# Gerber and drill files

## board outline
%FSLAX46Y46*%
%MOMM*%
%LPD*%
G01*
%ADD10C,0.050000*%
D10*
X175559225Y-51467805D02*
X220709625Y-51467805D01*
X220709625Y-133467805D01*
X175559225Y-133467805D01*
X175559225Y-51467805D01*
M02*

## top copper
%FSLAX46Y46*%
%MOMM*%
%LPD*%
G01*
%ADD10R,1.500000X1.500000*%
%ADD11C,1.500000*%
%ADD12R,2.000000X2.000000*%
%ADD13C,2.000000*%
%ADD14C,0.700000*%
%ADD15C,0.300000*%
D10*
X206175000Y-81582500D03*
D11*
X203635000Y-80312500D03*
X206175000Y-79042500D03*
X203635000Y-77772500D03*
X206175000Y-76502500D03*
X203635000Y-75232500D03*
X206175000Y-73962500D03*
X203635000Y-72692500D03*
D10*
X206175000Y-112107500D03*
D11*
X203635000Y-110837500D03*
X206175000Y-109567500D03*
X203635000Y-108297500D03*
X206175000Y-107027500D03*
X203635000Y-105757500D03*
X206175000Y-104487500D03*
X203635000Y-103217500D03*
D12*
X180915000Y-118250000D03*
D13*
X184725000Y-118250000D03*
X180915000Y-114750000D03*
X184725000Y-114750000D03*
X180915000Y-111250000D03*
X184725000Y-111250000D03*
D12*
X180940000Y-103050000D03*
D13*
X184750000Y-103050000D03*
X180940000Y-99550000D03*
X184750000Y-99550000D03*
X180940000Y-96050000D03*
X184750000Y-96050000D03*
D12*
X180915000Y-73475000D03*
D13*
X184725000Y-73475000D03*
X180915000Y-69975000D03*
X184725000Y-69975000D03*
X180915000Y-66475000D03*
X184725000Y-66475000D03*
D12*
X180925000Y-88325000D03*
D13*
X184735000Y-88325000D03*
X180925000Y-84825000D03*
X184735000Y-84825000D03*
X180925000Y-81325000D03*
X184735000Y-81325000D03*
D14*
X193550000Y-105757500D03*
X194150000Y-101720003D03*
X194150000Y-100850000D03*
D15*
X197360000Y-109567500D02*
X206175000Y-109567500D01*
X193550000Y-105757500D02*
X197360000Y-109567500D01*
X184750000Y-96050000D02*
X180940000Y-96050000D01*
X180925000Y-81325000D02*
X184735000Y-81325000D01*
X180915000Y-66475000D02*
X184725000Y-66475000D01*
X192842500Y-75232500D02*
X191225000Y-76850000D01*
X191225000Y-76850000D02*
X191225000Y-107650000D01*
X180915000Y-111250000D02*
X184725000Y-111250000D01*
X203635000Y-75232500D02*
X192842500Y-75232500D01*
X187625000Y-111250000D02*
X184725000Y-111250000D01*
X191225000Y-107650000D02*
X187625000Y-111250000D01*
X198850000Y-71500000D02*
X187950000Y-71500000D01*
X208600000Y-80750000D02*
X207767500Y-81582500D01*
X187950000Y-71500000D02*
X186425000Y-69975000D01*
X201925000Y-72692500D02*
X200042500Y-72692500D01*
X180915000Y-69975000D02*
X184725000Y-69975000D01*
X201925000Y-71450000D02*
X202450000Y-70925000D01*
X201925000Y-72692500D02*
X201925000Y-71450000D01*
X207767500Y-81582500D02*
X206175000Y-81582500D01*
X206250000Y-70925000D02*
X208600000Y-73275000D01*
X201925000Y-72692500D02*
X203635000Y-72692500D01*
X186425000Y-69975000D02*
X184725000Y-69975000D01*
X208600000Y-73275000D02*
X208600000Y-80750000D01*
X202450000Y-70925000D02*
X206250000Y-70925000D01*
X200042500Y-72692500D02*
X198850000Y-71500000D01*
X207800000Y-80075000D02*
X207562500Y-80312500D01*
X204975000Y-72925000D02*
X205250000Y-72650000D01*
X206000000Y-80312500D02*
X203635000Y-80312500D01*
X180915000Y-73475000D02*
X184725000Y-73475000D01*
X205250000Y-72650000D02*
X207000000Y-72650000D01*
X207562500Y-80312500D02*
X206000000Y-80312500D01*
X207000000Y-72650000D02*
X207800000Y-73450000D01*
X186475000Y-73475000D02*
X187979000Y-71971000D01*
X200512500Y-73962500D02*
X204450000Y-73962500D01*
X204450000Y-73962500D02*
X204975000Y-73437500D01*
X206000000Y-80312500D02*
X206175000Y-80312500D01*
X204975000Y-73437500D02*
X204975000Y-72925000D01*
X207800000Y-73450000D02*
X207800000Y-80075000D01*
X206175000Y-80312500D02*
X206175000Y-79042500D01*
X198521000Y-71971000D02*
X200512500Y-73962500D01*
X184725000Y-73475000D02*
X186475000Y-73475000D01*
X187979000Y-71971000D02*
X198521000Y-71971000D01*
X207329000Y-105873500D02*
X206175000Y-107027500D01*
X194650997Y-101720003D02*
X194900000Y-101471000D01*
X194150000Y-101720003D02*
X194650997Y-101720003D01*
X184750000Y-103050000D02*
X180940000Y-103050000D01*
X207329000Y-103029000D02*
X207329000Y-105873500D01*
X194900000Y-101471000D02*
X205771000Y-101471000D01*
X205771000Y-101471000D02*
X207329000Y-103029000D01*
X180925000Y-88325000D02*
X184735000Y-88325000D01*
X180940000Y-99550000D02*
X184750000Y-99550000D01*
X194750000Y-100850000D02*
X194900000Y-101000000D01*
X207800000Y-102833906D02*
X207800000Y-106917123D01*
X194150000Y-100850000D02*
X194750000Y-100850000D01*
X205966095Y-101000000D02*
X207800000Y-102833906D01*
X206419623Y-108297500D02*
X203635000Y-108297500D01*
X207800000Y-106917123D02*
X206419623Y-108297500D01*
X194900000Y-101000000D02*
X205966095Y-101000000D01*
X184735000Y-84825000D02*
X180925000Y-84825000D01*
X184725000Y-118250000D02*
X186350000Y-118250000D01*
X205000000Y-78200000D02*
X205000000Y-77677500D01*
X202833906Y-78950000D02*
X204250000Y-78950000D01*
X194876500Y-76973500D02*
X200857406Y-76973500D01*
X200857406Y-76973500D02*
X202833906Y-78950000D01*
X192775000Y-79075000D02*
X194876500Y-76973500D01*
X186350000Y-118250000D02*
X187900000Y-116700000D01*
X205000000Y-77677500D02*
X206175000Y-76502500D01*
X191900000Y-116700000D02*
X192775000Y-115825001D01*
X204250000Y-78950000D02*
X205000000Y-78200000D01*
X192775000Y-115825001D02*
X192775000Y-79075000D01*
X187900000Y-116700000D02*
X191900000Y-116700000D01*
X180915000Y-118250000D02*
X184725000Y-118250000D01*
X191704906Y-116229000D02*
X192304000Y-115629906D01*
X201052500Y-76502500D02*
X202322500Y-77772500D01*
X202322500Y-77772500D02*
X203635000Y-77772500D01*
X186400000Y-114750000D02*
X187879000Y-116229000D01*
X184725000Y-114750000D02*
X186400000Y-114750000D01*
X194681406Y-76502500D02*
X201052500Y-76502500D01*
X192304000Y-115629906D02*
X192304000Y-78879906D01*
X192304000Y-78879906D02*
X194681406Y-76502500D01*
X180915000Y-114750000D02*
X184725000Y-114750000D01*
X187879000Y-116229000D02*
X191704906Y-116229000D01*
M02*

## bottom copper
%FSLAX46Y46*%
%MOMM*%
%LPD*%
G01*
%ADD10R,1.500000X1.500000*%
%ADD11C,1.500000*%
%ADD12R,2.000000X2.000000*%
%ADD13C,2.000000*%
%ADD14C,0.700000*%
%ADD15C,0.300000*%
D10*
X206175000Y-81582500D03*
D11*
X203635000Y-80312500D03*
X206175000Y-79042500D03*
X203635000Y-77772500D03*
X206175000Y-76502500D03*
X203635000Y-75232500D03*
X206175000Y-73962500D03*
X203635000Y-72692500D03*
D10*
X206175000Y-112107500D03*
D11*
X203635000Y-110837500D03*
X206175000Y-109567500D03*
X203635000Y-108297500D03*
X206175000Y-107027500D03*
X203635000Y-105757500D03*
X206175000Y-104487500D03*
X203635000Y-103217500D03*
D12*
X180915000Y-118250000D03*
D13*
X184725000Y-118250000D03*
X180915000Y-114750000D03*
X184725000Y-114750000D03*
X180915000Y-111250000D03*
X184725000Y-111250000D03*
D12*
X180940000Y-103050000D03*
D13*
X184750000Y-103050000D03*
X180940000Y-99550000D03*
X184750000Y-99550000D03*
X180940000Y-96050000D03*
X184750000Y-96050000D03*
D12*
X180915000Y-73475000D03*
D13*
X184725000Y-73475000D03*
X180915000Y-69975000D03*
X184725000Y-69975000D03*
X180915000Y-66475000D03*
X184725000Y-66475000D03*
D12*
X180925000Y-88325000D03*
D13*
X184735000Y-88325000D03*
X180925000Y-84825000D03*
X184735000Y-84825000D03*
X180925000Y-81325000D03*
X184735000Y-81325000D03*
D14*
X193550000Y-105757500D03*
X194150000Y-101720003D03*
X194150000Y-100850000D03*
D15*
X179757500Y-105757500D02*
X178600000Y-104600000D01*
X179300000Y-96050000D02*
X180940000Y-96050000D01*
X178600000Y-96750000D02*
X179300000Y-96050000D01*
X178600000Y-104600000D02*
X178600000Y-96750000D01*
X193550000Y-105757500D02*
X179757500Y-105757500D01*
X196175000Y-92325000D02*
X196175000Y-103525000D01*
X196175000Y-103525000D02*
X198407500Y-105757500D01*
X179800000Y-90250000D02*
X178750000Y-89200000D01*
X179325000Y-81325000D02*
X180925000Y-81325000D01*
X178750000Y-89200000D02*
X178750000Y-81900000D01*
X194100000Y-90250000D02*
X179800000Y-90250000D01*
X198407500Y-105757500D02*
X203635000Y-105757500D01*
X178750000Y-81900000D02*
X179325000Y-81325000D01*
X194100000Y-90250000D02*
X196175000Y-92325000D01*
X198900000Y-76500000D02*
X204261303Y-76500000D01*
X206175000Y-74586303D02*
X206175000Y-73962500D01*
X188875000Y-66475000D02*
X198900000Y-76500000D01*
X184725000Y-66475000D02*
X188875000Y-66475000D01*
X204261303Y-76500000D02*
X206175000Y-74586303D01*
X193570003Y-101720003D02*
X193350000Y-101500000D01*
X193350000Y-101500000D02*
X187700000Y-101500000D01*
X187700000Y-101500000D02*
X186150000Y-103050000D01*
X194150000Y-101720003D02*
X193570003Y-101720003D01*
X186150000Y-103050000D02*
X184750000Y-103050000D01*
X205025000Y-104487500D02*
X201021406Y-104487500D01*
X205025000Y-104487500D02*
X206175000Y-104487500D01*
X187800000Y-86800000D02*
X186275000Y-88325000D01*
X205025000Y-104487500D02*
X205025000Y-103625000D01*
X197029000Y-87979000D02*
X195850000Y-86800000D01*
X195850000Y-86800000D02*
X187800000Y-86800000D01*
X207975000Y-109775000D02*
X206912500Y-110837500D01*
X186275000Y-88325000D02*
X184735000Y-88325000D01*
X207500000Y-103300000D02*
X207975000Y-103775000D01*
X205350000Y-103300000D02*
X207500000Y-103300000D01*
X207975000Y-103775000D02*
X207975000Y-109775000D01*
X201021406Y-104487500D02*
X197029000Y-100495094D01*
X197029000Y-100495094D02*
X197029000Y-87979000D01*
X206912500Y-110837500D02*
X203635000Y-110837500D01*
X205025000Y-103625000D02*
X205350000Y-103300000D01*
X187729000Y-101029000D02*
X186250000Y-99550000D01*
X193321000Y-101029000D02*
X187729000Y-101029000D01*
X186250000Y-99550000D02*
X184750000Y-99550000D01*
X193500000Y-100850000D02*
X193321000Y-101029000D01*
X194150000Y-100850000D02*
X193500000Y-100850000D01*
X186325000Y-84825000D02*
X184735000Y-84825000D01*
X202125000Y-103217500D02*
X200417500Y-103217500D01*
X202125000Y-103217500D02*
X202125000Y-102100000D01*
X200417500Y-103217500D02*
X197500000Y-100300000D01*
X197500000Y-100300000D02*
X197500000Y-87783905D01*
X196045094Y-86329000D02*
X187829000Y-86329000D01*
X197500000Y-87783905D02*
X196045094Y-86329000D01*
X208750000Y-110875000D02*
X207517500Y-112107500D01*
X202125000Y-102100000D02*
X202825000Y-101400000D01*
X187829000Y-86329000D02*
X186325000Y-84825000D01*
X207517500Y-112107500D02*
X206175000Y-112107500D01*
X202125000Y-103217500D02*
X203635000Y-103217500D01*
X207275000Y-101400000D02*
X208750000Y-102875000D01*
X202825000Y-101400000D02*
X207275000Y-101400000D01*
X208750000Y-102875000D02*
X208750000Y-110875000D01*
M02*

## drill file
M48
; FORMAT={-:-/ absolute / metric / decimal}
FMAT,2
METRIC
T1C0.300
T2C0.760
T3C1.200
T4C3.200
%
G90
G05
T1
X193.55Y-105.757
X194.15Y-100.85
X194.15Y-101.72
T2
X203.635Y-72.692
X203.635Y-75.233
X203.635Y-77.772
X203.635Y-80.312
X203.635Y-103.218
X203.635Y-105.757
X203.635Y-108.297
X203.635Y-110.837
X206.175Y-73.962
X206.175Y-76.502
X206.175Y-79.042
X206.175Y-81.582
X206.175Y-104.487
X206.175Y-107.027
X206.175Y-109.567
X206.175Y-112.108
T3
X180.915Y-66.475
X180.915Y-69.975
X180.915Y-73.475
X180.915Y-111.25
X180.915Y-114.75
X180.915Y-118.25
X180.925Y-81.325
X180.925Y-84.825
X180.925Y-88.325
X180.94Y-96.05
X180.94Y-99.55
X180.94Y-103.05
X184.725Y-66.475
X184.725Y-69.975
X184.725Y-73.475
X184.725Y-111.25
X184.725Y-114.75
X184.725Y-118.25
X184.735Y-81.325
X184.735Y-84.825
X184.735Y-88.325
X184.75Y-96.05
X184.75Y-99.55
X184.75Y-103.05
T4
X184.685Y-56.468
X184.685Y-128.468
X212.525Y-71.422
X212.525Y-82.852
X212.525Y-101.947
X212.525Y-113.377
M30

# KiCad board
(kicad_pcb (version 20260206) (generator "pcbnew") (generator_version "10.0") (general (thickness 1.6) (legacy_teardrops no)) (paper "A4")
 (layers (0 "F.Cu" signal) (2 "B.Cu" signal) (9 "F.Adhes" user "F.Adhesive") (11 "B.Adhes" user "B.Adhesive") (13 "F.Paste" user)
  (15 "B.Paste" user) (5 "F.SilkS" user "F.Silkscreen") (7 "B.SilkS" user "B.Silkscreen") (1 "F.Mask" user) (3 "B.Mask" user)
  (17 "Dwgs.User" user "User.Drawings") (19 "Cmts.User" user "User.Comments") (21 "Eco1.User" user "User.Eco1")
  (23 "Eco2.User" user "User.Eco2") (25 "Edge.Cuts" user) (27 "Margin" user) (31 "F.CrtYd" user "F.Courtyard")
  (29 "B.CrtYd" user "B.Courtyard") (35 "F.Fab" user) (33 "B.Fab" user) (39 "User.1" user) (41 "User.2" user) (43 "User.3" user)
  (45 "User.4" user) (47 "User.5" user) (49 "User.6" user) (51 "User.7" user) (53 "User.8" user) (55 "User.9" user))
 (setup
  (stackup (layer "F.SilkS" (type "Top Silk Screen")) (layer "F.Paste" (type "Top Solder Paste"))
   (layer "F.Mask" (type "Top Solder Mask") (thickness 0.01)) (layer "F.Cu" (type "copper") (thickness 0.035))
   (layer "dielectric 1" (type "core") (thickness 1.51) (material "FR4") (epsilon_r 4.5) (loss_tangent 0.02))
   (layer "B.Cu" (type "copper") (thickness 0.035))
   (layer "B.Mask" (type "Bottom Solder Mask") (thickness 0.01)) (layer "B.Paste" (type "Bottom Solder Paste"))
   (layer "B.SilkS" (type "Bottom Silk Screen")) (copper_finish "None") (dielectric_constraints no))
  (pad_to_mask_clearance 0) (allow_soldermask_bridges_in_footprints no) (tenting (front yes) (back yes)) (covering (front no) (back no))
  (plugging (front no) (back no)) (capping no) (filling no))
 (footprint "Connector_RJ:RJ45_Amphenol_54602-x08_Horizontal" (layer "F.Cu") (at 206.175 81.5825 90)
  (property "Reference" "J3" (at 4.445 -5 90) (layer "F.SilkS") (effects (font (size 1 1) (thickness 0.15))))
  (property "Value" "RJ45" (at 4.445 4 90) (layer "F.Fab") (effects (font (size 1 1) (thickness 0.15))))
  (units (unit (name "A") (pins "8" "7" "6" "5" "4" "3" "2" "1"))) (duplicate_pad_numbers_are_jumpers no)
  (pad "" np_thru_hole circle (at -1.27 6.35 90) (size 3.2 3.2) (drill 3.2) (layers "*.Cu" "*.Mask"))
  (pad "" np_thru_hole circle (at 10.16 6.35 90) (size 3.2 3.2) (drill 3.2) (layers "*.Cu" "*.Mask"))
  (pad "1" thru_hole rect (at 0 0 90) (size 1.5 1.5) (drill 0.76) (layers "*.Cu" "*.Mask") (remove_unused_layers no) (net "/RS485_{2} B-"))
  (pad "2" thru_hole circle (at 1.27 -2.54 90) (size 1.5 1.5) (drill 0.76) (layers "*.Cu" "*.Mask") (remove_unused_layers no)
   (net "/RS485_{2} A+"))
  (pad "3" thru_hole circle (at 2.54 0 90) (size 1.5 1.5) (drill 0.76) (layers "*.Cu" "*.Mask") (remove_unused_layers no)
   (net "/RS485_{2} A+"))
  (pad "4" thru_hole circle (at 3.81 -2.54 90) (size 1.5 1.5) (drill 0.76) (layers "*.Cu" "*.Mask") (remove_unused_layers no)
   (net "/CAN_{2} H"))
  (pad "5" thru_hole circle (at 5.08 0 90) (size 1.5 1.5) (drill 0.76) (layers "*.Cu" "*.Mask") (remove_unused_layers no) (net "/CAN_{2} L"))
  (pad "6" thru_hole circle (at 6.35 -2.54 90) (size 1.5 1.5) (drill 0.76) (layers "*.Cu" "*.Mask") (remove_unused_layers no)
   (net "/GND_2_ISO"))
  (pad "7" thru_hole circle (at 7.62 0 90) (size 1.5 1.5) (drill 0.76) (layers "*.Cu" "*.Mask") (remove_unused_layers no) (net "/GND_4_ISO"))
  (pad "8" thru_hole circle (at 8.89 -2.54 90) (size 1.5 1.5) (drill 0.76) (layers "*.Cu" "*.Mask") (remove_unused_layers no)
   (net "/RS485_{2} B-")))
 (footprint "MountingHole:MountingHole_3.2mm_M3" (layer "F.Cu") (at 184.684625 56.467805)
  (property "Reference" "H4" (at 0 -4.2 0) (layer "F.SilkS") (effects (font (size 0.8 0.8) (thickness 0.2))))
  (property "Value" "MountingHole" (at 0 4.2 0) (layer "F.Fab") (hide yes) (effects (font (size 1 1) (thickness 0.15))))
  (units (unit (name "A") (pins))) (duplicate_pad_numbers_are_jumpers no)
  (pad "" np_thru_hole circle (at 0 0) (size 3.2 3.2) (drill 3.2) (layers "*.Cu" "*.Mask")))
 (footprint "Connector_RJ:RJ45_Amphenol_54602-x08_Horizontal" (layer "F.Cu") (at 206.175 112.1075 90)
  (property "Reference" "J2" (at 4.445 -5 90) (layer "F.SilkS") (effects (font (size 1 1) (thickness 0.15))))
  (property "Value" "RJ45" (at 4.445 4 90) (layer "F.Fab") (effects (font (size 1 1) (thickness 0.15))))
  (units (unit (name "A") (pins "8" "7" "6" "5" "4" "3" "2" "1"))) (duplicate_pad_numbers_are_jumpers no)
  (pad "" np_thru_hole circle (at -1.27 6.35 90) (size 3.2 3.2) (drill 3.2) (layers "*.Cu" "*.Mask"))
  (pad "" np_thru_hole circle (at 10.16 6.35 90) (size 3.2 3.2) (drill 3.2) (layers "*.Cu" "*.Mask"))
  (pad "1" thru_hole rect (at 0 0 90) (size 1.5 1.5) (drill 0.76) (layers "*.Cu" "*.Mask") (remove_unused_layers no) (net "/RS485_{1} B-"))
  (pad "2" thru_hole circle (at 1.27 -2.54 90) (size 1.5 1.5) (drill 0.76) (layers "*.Cu" "*.Mask") (remove_unused_layers no)
   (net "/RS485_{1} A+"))
  (pad "3" thru_hole circle (at 2.54 0 90) (size 1.5 1.5) (drill 0.76) (layers "*.Cu" "*.Mask") (remove_unused_layers no) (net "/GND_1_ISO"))
  (pad "4" thru_hole circle (at 3.81 -2.54 90) (size 1.5 1.5) (drill 0.76) (layers "*.Cu" "*.Mask") (remove_unused_layers no)
   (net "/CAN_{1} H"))
  (pad "5" thru_hole circle (at 5.08 0 90) (size 1.5 1.5) (drill 0.76) (layers "*.Cu" "*.Mask") (remove_unused_layers no) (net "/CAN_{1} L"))
  (pad "6" thru_hole circle (at 6.35 -2.54 90) (size 1.5 1.5) (drill 0.76) (layers "*.Cu" "*.Mask") (remove_unused_layers no)
   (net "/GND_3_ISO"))
  (pad "7" thru_hole circle (at 7.62 0 90) (size 1.5 1.5) (drill 0.76) (layers "*.Cu" "*.Mask") (remove_unused_layers no)
   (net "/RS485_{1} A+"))
  (pad "8" thru_hole circle (at 8.89 -2.54 90) (size 1.5 1.5) (drill 0.76) (layers "*.Cu" "*.Mask") (remove_unused_layers no)
   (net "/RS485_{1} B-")))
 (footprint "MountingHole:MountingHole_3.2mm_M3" (layer "F.Cu") (at 184.684625 128.467805)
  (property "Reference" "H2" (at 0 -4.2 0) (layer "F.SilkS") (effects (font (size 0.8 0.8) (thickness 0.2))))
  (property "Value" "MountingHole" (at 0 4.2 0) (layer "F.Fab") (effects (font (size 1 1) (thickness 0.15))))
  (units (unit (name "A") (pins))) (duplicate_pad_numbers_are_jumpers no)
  (pad "" np_thru_hole circle (at 0 0) (size 3.2 3.2) (drill 3.2) (layers "*.Cu" "*.Mask")))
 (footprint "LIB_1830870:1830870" (layer "B.Cu") (at 180.915 118.25 90)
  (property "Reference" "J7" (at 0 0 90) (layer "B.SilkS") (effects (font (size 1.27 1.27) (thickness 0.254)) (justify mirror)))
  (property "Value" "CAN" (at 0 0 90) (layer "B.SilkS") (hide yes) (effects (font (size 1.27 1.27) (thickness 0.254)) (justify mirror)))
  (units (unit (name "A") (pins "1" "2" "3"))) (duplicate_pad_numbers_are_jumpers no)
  (pad "1" thru_hole rect (at 0 0 90) (size 2 2) (drill 1.2) (layers "*.Cu" "*.Mask") (remove_unused_layers no) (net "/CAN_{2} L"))
  (pad "1" thru_hole circle (at 0 3.81 90) (size 2 2) (drill 1.2) (layers "*.Cu" "*.Mask") (remove_unused_layers no) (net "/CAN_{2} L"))
  (pad "2" thru_hole circle (at 3.5 0 90) (size 2 2) (drill 1.2) (layers "*.Cu" "*.Mask") (remove_unused_layers no) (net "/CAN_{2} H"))
  (pad "2" thru_hole circle (at 3.5 3.81 90) (size 2 2) (drill 1.2) (layers "*.Cu" "*.Mask") (remove_unused_layers no) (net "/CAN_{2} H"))
  (pad "3" thru_hole circle (at 7 0 90) (size 2 2) (drill 1.2) (layers "*.Cu" "*.Mask") (remove_unused_layers no) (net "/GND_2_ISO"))
  (pad "3" thru_hole circle (at 7 3.81 90) (size 2 2) (drill 1.2) (layers "*.Cu" "*.Mask") (remove_unused_layers no) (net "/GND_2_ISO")))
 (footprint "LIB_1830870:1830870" (layer "B.Cu") (at 180.94 103.05 90)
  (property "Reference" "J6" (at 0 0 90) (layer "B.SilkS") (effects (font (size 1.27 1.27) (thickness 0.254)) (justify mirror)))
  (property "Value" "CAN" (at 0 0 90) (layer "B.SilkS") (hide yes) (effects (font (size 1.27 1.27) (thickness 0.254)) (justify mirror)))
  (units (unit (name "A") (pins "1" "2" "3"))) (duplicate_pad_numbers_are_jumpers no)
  (pad "1" thru_hole rect (at 0 0 90) (size 2 2) (drill 1.2) (layers "*.Cu" "*.Mask") (remove_unused_layers no) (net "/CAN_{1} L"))
  (pad "1" thru_hole circle (at 0 3.81 90) (size 2 2) (drill 1.2) (layers "*.Cu" "*.Mask") (remove_unused_layers no) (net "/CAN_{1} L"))
  (pad "2" thru_hole circle (at 3.5 0 90) (size 2 2) (drill 1.2) (layers "*.Cu" "*.Mask") (remove_unused_layers no) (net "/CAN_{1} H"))
  (pad "2" thru_hole circle (at 3.5 3.81 90) (size 2 2) (drill 1.2) (layers "*.Cu" "*.Mask") (remove_unused_layers no) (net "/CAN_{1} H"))
  (pad "3" thru_hole circle (at 7 0 90) (size 2 2) (drill 1.2) (layers "*.Cu" "*.Mask") (remove_unused_layers no) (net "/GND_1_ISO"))
  (pad "3" thru_hole circle (at 7 3.81 90) (size 2 2) (drill 1.2) (layers "*.Cu" "*.Mask") (remove_unused_layers no) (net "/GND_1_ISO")))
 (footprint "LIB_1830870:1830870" (layer "B.Cu") (at 180.915 73.475 90)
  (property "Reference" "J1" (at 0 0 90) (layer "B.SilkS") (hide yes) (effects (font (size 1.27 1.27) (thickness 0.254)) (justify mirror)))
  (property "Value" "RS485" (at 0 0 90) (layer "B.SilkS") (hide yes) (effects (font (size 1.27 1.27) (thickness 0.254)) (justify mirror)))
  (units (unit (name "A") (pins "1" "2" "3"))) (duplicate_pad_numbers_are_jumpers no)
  (pad "1" thru_hole rect (at 0 0 90) (size 2 2) (drill 1.2) (layers "*.Cu" "*.Mask") (remove_unused_layers no) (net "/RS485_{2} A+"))
  (pad "1" thru_hole circle (at 0 3.81 90) (size 2 2) (drill 1.2) (layers "*.Cu" "*.Mask") (remove_unused_layers no) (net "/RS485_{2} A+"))
  (pad "2" thru_hole circle (at 3.5 0 90) (size 2 2) (drill 1.2) (layers "*.Cu" "*.Mask") (remove_unused_layers no) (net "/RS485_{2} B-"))
  (pad "2" thru_hole circle (at 3.5 3.81 90) (size 2 2) (drill 1.2) (layers "*.Cu" "*.Mask") (remove_unused_layers no) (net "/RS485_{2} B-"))
  (pad "3" thru_hole circle (at 7 0 90) (size 2 2) (drill 1.2) (layers "*.Cu" "*.Mask") (remove_unused_layers no) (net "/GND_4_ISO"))
  (pad "3" thru_hole circle (at 7 3.81 90) (size 2 2) (drill 1.2) (layers "*.Cu" "*.Mask") (remove_unused_layers no) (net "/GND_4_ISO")))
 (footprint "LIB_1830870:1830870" (layer "B.Cu") (at 180.925 88.325 90)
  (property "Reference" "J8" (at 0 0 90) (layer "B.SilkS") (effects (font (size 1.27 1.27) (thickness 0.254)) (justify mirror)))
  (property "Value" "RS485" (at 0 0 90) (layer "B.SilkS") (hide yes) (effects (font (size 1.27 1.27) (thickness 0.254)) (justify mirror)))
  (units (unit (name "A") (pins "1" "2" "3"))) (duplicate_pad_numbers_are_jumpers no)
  (pad "1" thru_hole rect (at 0 0 90) (size 2 2) (drill 1.2) (layers "*.Cu" "*.Mask") (remove_unused_layers no) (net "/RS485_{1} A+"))
  (pad "1" thru_hole circle (at 0 3.81 90) (size 2 2) (drill 1.2) (layers "*.Cu" "*.Mask") (remove_unused_layers no) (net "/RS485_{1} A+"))
  (pad "2" thru_hole circle (at 3.5 0 90) (size 2 2) (drill 1.2) (layers "*.Cu" "*.Mask") (remove_unused_layers no) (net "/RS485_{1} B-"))
  (pad "2" thru_hole circle (at 3.5 3.81 90) (size 2 2) (drill 1.2) (layers "*.Cu" "*.Mask") (remove_unused_layers no) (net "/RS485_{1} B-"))
  (pad "3" thru_hole circle (at 7 0 90) (size 2 2) (drill 1.2) (layers "*.Cu" "*.Mask") (remove_unused_layers no) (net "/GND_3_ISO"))
  (pad "3" thru_hole circle (at 7 3.81 90) (size 2 2) (drill 1.2) (layers "*.Cu" "*.Mask") (remove_unused_layers no) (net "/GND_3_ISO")))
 (gr_rect (start 175.559225 51.467805) (end 220.709625 133.467805) (stroke (width 0.05) (type default)) (fill no) (layer "Edge.Cuts"))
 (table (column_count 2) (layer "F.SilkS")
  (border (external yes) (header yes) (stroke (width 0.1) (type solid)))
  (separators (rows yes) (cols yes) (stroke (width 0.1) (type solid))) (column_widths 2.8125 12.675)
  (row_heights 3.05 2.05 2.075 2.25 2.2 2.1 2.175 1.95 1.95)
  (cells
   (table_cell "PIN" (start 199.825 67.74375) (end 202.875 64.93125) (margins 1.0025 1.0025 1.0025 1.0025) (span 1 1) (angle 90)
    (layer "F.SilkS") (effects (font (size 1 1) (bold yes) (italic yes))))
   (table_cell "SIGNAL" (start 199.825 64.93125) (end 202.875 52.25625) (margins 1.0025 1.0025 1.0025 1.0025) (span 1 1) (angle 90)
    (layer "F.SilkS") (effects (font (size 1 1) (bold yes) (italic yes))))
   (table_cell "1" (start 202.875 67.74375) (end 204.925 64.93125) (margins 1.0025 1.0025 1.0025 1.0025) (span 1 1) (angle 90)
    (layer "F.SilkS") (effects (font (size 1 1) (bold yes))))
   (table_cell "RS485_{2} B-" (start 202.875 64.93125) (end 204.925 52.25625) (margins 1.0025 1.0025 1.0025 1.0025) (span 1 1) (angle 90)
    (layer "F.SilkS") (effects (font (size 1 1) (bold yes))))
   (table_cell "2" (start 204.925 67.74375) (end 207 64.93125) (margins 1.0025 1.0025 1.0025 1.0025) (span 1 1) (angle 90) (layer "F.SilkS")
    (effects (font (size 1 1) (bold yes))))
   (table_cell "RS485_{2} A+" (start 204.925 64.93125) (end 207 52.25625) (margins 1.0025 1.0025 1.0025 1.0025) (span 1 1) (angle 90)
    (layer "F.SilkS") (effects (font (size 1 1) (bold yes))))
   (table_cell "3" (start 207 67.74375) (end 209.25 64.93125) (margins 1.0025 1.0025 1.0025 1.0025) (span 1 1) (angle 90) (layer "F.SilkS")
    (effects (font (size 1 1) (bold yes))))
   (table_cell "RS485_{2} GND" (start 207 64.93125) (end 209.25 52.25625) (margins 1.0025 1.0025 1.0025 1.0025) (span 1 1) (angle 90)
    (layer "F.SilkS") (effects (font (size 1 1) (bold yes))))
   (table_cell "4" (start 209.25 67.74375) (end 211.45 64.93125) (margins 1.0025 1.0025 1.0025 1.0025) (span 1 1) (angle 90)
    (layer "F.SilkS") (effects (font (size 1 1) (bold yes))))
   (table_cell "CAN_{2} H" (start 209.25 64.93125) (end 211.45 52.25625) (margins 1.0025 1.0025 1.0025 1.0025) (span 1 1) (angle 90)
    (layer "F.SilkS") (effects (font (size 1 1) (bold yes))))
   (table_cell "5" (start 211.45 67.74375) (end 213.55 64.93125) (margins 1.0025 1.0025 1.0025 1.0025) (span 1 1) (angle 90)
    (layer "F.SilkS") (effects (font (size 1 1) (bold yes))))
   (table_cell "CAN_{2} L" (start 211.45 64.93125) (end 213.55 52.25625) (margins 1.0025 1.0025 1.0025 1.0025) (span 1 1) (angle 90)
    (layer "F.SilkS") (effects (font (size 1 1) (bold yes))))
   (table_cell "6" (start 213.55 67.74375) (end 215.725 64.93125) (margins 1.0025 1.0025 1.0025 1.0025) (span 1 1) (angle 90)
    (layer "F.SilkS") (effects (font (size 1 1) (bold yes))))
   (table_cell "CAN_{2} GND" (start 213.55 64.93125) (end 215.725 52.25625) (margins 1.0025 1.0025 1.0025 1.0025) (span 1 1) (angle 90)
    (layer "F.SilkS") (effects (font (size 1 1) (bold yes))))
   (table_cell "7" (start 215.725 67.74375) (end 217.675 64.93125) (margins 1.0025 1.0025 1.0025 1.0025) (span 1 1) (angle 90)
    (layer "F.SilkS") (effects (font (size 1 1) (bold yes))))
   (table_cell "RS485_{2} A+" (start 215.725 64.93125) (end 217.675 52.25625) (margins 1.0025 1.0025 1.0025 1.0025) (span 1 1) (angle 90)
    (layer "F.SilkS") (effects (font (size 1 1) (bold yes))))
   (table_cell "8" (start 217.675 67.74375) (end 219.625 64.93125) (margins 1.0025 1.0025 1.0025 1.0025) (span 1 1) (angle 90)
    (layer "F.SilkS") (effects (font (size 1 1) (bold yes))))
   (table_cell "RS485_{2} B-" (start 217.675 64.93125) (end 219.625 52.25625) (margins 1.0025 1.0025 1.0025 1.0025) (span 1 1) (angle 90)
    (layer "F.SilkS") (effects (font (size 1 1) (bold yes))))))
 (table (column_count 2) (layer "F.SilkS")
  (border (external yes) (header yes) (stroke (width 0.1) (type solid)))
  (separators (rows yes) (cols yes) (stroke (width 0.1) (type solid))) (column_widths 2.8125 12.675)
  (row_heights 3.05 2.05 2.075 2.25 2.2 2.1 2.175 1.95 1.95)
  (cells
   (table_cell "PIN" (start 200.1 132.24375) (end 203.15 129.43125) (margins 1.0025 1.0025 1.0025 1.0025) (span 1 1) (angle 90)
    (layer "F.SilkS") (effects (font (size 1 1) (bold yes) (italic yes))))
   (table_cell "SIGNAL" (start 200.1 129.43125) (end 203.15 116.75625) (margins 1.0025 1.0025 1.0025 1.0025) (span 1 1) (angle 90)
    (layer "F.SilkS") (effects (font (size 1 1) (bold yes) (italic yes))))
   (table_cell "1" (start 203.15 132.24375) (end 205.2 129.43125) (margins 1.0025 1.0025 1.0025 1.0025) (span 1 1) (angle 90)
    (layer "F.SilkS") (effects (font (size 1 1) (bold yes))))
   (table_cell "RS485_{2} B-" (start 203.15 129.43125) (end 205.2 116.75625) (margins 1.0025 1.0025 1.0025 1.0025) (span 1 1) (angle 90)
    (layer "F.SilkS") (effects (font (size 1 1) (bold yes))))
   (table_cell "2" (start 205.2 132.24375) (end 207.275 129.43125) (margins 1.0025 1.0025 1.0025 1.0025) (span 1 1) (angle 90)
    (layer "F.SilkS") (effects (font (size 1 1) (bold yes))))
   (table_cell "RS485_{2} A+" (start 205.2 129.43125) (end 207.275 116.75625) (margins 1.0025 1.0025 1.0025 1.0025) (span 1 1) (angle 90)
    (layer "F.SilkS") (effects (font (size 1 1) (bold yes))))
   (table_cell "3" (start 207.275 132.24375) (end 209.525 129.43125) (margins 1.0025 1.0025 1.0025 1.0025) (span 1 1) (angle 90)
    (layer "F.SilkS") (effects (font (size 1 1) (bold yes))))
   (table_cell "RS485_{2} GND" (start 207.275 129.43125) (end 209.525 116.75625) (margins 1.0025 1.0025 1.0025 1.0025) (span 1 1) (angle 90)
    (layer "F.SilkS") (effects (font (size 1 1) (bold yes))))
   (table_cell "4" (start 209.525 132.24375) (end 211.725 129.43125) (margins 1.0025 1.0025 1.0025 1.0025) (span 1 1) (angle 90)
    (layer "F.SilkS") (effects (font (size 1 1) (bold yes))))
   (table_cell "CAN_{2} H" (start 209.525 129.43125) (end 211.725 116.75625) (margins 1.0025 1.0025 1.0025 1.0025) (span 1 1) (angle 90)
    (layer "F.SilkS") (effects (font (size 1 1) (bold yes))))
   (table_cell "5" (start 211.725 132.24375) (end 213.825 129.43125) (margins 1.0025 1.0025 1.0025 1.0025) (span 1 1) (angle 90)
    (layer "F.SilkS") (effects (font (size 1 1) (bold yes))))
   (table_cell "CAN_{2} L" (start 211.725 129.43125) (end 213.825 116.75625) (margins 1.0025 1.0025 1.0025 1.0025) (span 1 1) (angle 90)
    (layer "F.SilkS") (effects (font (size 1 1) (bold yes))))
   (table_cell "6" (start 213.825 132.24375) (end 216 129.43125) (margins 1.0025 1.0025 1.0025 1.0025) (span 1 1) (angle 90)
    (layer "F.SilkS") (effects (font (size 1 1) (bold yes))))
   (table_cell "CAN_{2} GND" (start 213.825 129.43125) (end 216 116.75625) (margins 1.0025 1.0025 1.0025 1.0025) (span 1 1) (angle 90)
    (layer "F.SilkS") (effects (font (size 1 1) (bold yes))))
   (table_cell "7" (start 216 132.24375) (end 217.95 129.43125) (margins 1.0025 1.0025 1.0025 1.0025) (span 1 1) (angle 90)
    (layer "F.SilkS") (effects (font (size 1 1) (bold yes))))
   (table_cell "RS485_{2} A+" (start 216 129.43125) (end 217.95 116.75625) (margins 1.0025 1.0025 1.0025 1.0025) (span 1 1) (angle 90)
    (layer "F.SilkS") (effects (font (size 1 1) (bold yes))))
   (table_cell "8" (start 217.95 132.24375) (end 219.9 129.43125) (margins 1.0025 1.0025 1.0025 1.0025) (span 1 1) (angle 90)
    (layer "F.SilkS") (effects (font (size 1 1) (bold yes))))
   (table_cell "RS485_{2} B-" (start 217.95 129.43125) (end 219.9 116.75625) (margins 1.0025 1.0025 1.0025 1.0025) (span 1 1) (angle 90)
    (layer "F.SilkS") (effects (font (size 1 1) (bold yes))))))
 (segment (start 197.36 109.5675) (end 206.175 109.5675) (width 0.3) (layer "F.Cu") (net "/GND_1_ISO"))
 (segment (start 193.55 105.7575) (end 197.36 109.5675) (width 0.3) (layer "F.Cu") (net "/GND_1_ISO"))
 (segment (start 184.75 96.05) (end 180.94 96.05) (width 0.3) (layer "F.Cu") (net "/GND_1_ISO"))
 (via (at 193.55 105.7575) (size 0.7) (drill 0.3) (layers "F.Cu" "B.Cu") (capping no) (covering (front no) (back no))
  (plugging (front no) (back no)) (filling no) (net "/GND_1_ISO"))
 (segment (start 179.7575 105.7575) (end 178.6 104.6) (width 0.3) (layer "B.Cu") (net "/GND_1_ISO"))
 (segment (start 179.3 96.05) (end 180.94 96.05) (width 0.3) (layer "B.Cu") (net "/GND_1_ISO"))
 (segment (start 178.6 96.75) (end 179.3 96.05) (width 0.3) (layer "B.Cu") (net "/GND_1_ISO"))
 (segment (start 178.6 104.6) (end 178.6 96.75) (width 0.3) (layer "B.Cu") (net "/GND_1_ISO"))
 (segment (start 193.55 105.7575) (end 179.7575 105.7575) (width 0.3) (layer "B.Cu") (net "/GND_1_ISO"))
 (segment (start 180.925 81.325) (end 184.735 81.325) (width 0.3) (layer "F.Cu") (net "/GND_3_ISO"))
 (segment (start 196.175 92.325) (end 196.175 103.525) (width 0.3) (layer "B.Cu") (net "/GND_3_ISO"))
 (segment (start 196.175 103.525) (end 198.4075 105.7575) (width 0.3) (layer "B.Cu") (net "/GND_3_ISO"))
 (segment (start 179.8 90.25) (end 178.75 89.2) (width 0.3) (layer "B.Cu") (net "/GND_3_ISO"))
 (segment (start 179.325 81.325) (end 180.925 81.325) (width 0.3) (layer "B.Cu") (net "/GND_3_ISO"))
 (segment (start 178.75 89.2) (end 178.75 81.9) (width 0.3) (layer "B.Cu") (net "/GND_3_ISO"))
 (segment (start 194.1 90.25) (end 179.8 90.25) (width 0.3) (layer "B.Cu") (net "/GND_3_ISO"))
 (segment (start 198.4075 105.7575) (end 203.635 105.7575) (width 0.3) (layer "B.Cu") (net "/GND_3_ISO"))
 (segment (start 178.75 81.9) (end 179.325 81.325) (width 0.3) (layer "B.Cu") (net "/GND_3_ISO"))
 (segment (start 194.1 90.25) (end 196.175 92.325) (width 0.3) (layer "B.Cu") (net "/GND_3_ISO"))
 (segment (start 180.915 66.475) (end 184.725 66.475) (width 0.3) (layer "F.Cu") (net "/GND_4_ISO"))
 (segment (start 198.9 76.5) (end 204.261303 76.5) (width 0.3) (layer "B.Cu") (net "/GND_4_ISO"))
 (segment (start 206.175 74.586303) (end 206.175 73.9625) (width 0.3) (layer "B.Cu") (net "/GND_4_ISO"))
 (segment (start 188.875 66.475) (end 198.9 76.5) (width 0.3) (layer "B.Cu") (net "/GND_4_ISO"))
 (segment (start 184.725 66.475) (end 188.875 66.475) (width 0.3) (layer "B.Cu") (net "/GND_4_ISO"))
 (segment (start 204.261303 76.5) (end 206.175 74.586303) (width 0.3) (layer "B.Cu") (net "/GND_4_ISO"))
 (segment (start 192.8425 75.2325) (end 191.225 76.85) (width 0.3) (layer "F.Cu") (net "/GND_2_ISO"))
 (segment (start 191.225 76.85) (end 191.225 107.65) (width 0.3) (layer "F.Cu") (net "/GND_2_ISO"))
 (segment (start 180.915 111.25) (end 184.725 111.25) (width 0.3) (layer "F.Cu") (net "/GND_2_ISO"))
 (segment (start 203.635 75.2325) (end 192.8425 75.2325) (width 0.3) (layer "F.Cu") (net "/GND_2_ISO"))
 (segment (start 187.625 111.25) (end 184.725 111.25) (width 0.3) (layer "F.Cu") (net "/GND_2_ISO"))
 (segment (start 191.225 107.65) (end 187.625 111.25) (width 0.3) (layer "F.Cu") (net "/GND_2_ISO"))
 (segment (start 198.85 71.5) (end 187.95 71.5) (width 0.3) (layer "F.Cu") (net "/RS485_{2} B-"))
 (segment (start 208.6 80.75) (end 207.7675 81.5825) (width 0.3) (layer "F.Cu") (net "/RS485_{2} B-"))
 (segment (start 187.95 71.5) (end 186.425 69.975) (width 0.3) (layer "F.Cu") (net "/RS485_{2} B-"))
 (segment (start 201.925 72.6925) (end 200.0425 72.6925) (width 0.3) (layer "F.Cu") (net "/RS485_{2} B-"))
 (segment (start 180.915 69.975) (end 184.725 69.975) (width 0.3) (layer "F.Cu") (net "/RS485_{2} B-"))
 (segment (start 201.925 71.45) (end 202.45 70.925) (width 0.3) (layer "F.Cu") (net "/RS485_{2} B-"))
 (segment (start 201.925 72.6925) (end 201.925 71.45) (width 0.3) (layer "F.Cu") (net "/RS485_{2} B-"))
 (segment (start 207.7675 81.5825) (end 206.175 81.5825) (width 0.3) (layer "F.Cu") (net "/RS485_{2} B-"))
 (segment (start 206.25 70.925) (end 208.6 73.275) (width 0.3) (layer "F.Cu") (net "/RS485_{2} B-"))
 (segment (start 201.925 72.6925) (end 203.635 72.6925) (width 0.3) (layer "F.Cu") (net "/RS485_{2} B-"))
 (segment (start 186.425 69.975) (end 184.725 69.975) (width 0.3) (layer "F.Cu") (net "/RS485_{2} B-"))
 (segment (start 208.6 73.275) (end 208.6 80.75) (width 0.3) (layer "F.Cu") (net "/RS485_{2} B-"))
 (segment (start 202.45 70.925) (end 206.25 70.925) (width 0.3) (layer "F.Cu") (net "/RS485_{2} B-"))
 (segment (start 200.0425 72.6925) (end 198.85 71.5) (width 0.3) (layer "F.Cu") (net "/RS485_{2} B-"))
 (segment (start 207.8 80.075) (end 207.5625 80.3125) (width 0.3) (layer "F.Cu") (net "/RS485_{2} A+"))
 (segment (start 204.975 72.925) (end 205.25 72.65) (width 0.3) (layer "F.Cu") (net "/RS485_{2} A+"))
 (segment (start 206 80.3125) (end 203.635 80.3125) (width 0.3) (layer "F.Cu") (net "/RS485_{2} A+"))
 (segment (start 180.915 73.475) (end 184.725 73.475) (width 0.3) (layer "F.Cu") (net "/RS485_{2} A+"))
 (segment (start 205.25 72.65) (end 207 72.65) (width 0.3) (layer "F.Cu") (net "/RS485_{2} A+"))
 (segment (start 207.5625 80.3125) (end 206 80.3125) (width 0.3) (layer "F.Cu") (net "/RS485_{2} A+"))
 (segment (start 207 72.65) (end 207.8 73.45) (width 0.3) (layer "F.Cu") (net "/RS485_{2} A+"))
 (segment (start 186.475 73.475) (end 187.979 71.971) (width 0.3) (layer "F.Cu") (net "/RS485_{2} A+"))
 (segment (start 200.5125 73.9625) (end 204.45 73.9625) (width 0.3) (layer "F.Cu") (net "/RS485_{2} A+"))
 (segment (start 204.45 73.9625) (end 204.975 73.4375) (width 0.3) (layer "F.Cu") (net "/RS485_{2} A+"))
 (segment (start 206 80.3125) (end 206.175 80.3125) (width 0.3) (layer "F.Cu") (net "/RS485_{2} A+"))
 (segment (start 204.975 73.4375) (end 204.975 72.925) (width 0.3) (layer "F.Cu") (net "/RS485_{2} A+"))
 (segment (start 207.8 73.45) (end 207.8 80.075) (width 0.3) (layer "F.Cu") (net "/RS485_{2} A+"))
 (segment (start 206.175 80.3125) (end 206.175 79.0425) (width 0.3) (layer "F.Cu") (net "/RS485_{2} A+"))
 (segment (start 198.521 71.971) (end 200.5125 73.9625) (width 0.3) (layer "F.Cu") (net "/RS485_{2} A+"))
 (segment (start 184.725 73.475) (end 186.475 73.475) (width 0.3) (layer "F.Cu") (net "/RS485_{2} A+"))
 (segment (start 187.979 71.971) (end 198.521 71.971) (width 0.3) (layer "F.Cu") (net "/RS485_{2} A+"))
 (segment (start 207.329 105.8735) (end 206.175 107.0275) (width 0.3) (layer "F.Cu") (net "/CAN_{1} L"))
 (segment (start 194.650997 101.720003) (end 194.9 101.471) (width 0.3) (layer "F.Cu") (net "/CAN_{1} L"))
 (segment (start 194.15 101.720003) (end 194.650997 101.720003) (width 0.3) (layer "F.Cu") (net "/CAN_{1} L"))
 (segment (start 184.75 103.05) (end 180.94 103.05) (width 0.3) (layer "F.Cu") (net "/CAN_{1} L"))
 (segment (start 207.329 103.029) (end 207.329 105.8735) (width 0.3) (layer "F.Cu") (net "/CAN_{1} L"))
 (segment (start 194.9 101.471) (end 205.771 101.471) (width 0.3) (layer "F.Cu") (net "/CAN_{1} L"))
 (segment (start 205.771 101.471) (end 207.329 103.029) (width 0.3) (layer "F.Cu") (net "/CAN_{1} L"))
 (via (at 194.15 101.720003) (size 0.7) (drill 0.3) (layers "F.Cu" "B.Cu") (capping no) (covering (front no) (back no))
  (plugging (front no) (back no)) (filling no) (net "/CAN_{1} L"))
 (segment (start 193.570003 101.720003) (end 193.35 101.5) (width 0.3) (layer "B.Cu") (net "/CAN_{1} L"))
 (segment (start 193.35 101.5) (end 187.7 101.5) (width 0.3) (layer "B.Cu") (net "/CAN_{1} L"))
 (segment (start 187.7 101.5) (end 186.15 103.05) (width 0.3) (layer "B.Cu") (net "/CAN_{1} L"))
 (segment (start 194.15 101.720003) (end 193.570003 101.720003) (width 0.3) (layer "B.Cu") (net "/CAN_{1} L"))
 (segment (start 186.15 103.05) (end 184.75 103.05) (width 0.3) (layer "B.Cu") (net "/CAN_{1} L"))
 (segment (start 180.925 88.325) (end 184.735 88.325) (width 0.3) (layer "F.Cu") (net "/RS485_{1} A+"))
 (segment (start 205.025 104.4875) (end 201.021406 104.4875) (width 0.3) (layer "B.Cu") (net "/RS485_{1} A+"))
 (segment (start 205.025 104.4875) (end 206.175 104.4875) (width 0.3) (layer "B.Cu") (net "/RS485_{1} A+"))
 (segment (start 187.8 86.8) (end 186.275 88.325) (width 0.3) (layer "B.Cu") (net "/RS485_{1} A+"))
 (segment (start 205.025 104.4875) (end 205.025 103.625) (width 0.3) (layer "B.Cu") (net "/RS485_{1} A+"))
 (segment (start 197.029 87.979) (end 195.85 86.8) (width 0.3) (layer "B.Cu") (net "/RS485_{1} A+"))
 (segment (start 195.85 86.8) (end 187.8 86.8) (width 0.3) (layer "B.Cu") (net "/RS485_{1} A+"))
 (segment (start 207.975 109.775) (end 206.9125 110.8375) (width 0.3) (layer "B.Cu") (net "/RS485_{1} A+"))
 (segment (start 186.275 88.325) (end 184.735 88.325) (width 0.3) (layer "B.Cu") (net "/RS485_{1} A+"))
 (segment (start 207.5 103.3) (end 207.975 103.775) (width 0.3) (layer "B.Cu") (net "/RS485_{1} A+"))
 (segment (start 205.35 103.3) (end 207.5 103.3) (width 0.3) (layer "B.Cu") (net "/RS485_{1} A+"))
 (segment (start 207.975 103.775) (end 207.975 109.775) (width 0.3) (layer "B.Cu") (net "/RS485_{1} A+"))
 (segment (start 201.021406 104.4875) (end 197.029 100.495094) (width 0.3) (layer "B.Cu") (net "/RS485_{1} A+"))
 (segment (start 197.029 100.495094) (end 197.029 87.979) (width 0.3) (layer "B.Cu") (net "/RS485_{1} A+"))
 (segment (start 206.9125 110.8375) (end 203.635 110.8375) (width 0.3) (layer "B.Cu") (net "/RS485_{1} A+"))
 (segment (start 205.025 103.625) (end 205.35 103.3) (width 0.3) (layer "B.Cu") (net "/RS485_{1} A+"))
 (segment (start 180.94 99.55) (end 184.75 99.55) (width 0.3) (layer "F.Cu") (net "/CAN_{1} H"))
 (segment (start 194.75 100.85) (end 194.9 101) (width 0.3) (layer "F.Cu") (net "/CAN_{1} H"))
 (segment (start 207.8 102.833906) (end 207.8 106.917123) (width 0.3) (layer "F.Cu") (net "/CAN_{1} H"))
 (segment (start 194.15 100.85) (end 194.75 100.85) (width 0.3) (layer "F.Cu") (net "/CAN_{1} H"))
 (segment (start 205.966095 101) (end 207.8 102.833906) (width 0.3) (layer "F.Cu") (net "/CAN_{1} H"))
 (segment (start 206.419623 108.2975) (end 203.635 108.2975) (width 0.3) (layer "F.Cu") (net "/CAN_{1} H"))
 (segment (start 207.8 106.917123) (end 206.419623 108.2975) (width 0.3) (layer "F.Cu") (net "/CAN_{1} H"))
 (segment (start 194.9 101) (end 205.966095 101) (width 0.3) (layer "F.Cu") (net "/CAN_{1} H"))
 (via (at 194.15 100.85) (size 0.7) (drill 0.3) (layers "F.Cu" "B.Cu") (capping no) (covering (front no) (back no))
  (plugging (front no) (back no)) (filling no) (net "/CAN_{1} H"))
 (segment (start 187.729 101.029) (end 186.25 99.55) (width 0.3) (layer "B.Cu") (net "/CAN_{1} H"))
 (segment (start 193.321 101.029) (end 187.729 101.029) (width 0.3) (layer "B.Cu") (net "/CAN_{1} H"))
 (segment (start 186.25 99.55) (end 184.75 99.55) (width 0.3) (layer "B.Cu") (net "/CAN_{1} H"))
 (segment (start 193.5 100.85) (end 193.321 101.029) (width 0.3) (layer "B.Cu") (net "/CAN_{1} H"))
 (segment (start 194.15 100.85) (end 193.5 100.85) (width 0.3) (layer "B.Cu") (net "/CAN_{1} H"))
 (segment (start 184.735 84.825) (end 180.925 84.825) (width 0.3) (layer "F.Cu") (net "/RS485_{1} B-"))
 (segment (start 186.325 84.825) (end 184.735 84.825) (width 0.3) (layer "B.Cu") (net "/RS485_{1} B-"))
 (segment (start 202.125 103.2175) (end 200.4175 103.2175) (width 0.3) (layer "B.Cu") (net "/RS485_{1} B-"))
 (segment (start 202.125 103.2175) (end 202.125 102.1) (width 0.3) (layer "B.Cu") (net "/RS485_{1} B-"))
 (segment (start 200.4175 103.2175) (end 197.5 100.3) (width 0.3) (layer "B.Cu") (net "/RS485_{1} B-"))
 (segment (start 197.5 100.3) (end 197.5 87.783905) (width 0.3) (layer "B.Cu") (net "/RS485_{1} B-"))
 (segment (start 196.045094 86.329) (end 187.829 86.329) (width 0.3) (layer "B.Cu") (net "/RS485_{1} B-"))
 (segment (start 197.5 87.783905) (end 196.045094 86.329) (width 0.3) (layer "B.Cu") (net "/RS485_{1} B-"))
 (segment (start 208.75 110.875) (end 207.5175 112.1075) (width 0.3) (layer "B.Cu") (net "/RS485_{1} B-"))
 (segment (start 202.125 102.1) (end 202.825 101.4) (width 0.3) (layer "B.Cu") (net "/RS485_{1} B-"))
 (segment (start 187.829 86.329) (end 186.325 84.825) (width 0.3) (layer "B.Cu") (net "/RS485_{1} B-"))
 (segment (start 207.5175 112.1075) (end 206.175 112.1075) (width 0.3) (layer "B.Cu") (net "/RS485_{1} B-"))
 (segment (start 202.125 103.2175) (end 203.635 103.2175) (width 0.3) (layer "B.Cu") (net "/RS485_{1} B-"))
 (segment (start 207.275 101.4) (end 208.75 102.875) (width 0.3) (layer "B.Cu") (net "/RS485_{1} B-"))
 (segment (start 202.825 101.4) (end 207.275 101.4) (width 0.3) (layer "B.Cu") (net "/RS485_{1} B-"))
 (segment (start 208.75 102.875) (end 208.75 110.875) (width 0.3) (layer "B.Cu") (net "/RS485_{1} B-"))
 (segment (start 184.725 118.25) (end 186.35 118.25) (width 0.3) (layer "F.Cu") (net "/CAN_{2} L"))
 (segment (start 205 78.2) (end 205 77.6775) (width 0.3) (layer "F.Cu") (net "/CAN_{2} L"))
 (segment (start 202.833906 78.95) (end 204.25 78.95) (width 0.3) (layer "F.Cu") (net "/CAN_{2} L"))
 (segment (start 194.8765 76.9735) (end 200.857406 76.9735) (width 0.3) (layer "F.Cu") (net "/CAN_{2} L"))
 (segment (start 200.857406 76.9735) (end 202.833906 78.95) (width 0.3) (layer "F.Cu") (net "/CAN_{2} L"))
 (segment (start 192.775 79.075) (end 194.8765 76.9735) (width 0.3) (layer "F.Cu") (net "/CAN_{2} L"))
 (segment (start 186.35 118.25) (end 187.9 116.7) (width 0.3) (layer "F.Cu") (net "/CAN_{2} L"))
 (segment (start 205 77.6775) (end 206.175 76.5025) (width 0.3) (layer "F.Cu") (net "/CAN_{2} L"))
 (segment (start 191.9 116.7) (end 192.775 115.825001) (width 0.3) (layer "F.Cu") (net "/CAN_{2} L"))
 (segment (start 204.25 78.95) (end 205 78.2) (width 0.3) (layer "F.Cu") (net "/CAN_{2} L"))
 (segment (start 192.775 115.825001) (end 192.775 79.075) (width 0.3) (layer "F.Cu") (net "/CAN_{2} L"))
 (segment (start 187.9 116.7) (end 191.9 116.7) (width 0.3) (layer "F.Cu") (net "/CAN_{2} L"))
 (segment (start 180.915 118.25) (end 184.725 118.25) (width 0.3) (layer "F.Cu") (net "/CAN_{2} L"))
 (segment (start 191.704906 116.229) (end 192.304 115.629906) (width 0.3) (layer "F.Cu") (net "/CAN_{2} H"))
 (segment (start 201.0525 76.5025) (end 202.3225 77.7725) (width 0.3) (layer "F.Cu") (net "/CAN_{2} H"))
 (segment (start 202.3225 77.7725) (end 203.635 77.7725) (width 0.3) (layer "F.Cu") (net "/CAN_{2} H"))
 (segment (start 186.4 114.75) (end 187.879 116.229) (width 0.3) (layer "F.Cu") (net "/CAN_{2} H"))
 (segment (start 184.725 114.75) (end 186.4 114.75) (width 0.3) (layer "F.Cu") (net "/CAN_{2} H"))
 (segment (start 194.681406 76.5025) (end 201.0525 76.5025) (width 0.3) (layer "F.Cu") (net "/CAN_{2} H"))
 (segment (start 192.304 115.629906) (end 192.304 78.879906) (width 0.3) (layer "F.Cu") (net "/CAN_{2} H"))
 (segment (start 192.304 78.879906) (end 194.681406 76.5025) (width 0.3) (layer "F.Cu") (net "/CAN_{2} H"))
 (segment (start 180.915 114.75) (end 184.725 114.75) (width 0.3) (layer "F.Cu") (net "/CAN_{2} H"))
 (segment (start 187.879 116.229) (end 191.704906 116.229) (width 0.3) (layer "F.Cu") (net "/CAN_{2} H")))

